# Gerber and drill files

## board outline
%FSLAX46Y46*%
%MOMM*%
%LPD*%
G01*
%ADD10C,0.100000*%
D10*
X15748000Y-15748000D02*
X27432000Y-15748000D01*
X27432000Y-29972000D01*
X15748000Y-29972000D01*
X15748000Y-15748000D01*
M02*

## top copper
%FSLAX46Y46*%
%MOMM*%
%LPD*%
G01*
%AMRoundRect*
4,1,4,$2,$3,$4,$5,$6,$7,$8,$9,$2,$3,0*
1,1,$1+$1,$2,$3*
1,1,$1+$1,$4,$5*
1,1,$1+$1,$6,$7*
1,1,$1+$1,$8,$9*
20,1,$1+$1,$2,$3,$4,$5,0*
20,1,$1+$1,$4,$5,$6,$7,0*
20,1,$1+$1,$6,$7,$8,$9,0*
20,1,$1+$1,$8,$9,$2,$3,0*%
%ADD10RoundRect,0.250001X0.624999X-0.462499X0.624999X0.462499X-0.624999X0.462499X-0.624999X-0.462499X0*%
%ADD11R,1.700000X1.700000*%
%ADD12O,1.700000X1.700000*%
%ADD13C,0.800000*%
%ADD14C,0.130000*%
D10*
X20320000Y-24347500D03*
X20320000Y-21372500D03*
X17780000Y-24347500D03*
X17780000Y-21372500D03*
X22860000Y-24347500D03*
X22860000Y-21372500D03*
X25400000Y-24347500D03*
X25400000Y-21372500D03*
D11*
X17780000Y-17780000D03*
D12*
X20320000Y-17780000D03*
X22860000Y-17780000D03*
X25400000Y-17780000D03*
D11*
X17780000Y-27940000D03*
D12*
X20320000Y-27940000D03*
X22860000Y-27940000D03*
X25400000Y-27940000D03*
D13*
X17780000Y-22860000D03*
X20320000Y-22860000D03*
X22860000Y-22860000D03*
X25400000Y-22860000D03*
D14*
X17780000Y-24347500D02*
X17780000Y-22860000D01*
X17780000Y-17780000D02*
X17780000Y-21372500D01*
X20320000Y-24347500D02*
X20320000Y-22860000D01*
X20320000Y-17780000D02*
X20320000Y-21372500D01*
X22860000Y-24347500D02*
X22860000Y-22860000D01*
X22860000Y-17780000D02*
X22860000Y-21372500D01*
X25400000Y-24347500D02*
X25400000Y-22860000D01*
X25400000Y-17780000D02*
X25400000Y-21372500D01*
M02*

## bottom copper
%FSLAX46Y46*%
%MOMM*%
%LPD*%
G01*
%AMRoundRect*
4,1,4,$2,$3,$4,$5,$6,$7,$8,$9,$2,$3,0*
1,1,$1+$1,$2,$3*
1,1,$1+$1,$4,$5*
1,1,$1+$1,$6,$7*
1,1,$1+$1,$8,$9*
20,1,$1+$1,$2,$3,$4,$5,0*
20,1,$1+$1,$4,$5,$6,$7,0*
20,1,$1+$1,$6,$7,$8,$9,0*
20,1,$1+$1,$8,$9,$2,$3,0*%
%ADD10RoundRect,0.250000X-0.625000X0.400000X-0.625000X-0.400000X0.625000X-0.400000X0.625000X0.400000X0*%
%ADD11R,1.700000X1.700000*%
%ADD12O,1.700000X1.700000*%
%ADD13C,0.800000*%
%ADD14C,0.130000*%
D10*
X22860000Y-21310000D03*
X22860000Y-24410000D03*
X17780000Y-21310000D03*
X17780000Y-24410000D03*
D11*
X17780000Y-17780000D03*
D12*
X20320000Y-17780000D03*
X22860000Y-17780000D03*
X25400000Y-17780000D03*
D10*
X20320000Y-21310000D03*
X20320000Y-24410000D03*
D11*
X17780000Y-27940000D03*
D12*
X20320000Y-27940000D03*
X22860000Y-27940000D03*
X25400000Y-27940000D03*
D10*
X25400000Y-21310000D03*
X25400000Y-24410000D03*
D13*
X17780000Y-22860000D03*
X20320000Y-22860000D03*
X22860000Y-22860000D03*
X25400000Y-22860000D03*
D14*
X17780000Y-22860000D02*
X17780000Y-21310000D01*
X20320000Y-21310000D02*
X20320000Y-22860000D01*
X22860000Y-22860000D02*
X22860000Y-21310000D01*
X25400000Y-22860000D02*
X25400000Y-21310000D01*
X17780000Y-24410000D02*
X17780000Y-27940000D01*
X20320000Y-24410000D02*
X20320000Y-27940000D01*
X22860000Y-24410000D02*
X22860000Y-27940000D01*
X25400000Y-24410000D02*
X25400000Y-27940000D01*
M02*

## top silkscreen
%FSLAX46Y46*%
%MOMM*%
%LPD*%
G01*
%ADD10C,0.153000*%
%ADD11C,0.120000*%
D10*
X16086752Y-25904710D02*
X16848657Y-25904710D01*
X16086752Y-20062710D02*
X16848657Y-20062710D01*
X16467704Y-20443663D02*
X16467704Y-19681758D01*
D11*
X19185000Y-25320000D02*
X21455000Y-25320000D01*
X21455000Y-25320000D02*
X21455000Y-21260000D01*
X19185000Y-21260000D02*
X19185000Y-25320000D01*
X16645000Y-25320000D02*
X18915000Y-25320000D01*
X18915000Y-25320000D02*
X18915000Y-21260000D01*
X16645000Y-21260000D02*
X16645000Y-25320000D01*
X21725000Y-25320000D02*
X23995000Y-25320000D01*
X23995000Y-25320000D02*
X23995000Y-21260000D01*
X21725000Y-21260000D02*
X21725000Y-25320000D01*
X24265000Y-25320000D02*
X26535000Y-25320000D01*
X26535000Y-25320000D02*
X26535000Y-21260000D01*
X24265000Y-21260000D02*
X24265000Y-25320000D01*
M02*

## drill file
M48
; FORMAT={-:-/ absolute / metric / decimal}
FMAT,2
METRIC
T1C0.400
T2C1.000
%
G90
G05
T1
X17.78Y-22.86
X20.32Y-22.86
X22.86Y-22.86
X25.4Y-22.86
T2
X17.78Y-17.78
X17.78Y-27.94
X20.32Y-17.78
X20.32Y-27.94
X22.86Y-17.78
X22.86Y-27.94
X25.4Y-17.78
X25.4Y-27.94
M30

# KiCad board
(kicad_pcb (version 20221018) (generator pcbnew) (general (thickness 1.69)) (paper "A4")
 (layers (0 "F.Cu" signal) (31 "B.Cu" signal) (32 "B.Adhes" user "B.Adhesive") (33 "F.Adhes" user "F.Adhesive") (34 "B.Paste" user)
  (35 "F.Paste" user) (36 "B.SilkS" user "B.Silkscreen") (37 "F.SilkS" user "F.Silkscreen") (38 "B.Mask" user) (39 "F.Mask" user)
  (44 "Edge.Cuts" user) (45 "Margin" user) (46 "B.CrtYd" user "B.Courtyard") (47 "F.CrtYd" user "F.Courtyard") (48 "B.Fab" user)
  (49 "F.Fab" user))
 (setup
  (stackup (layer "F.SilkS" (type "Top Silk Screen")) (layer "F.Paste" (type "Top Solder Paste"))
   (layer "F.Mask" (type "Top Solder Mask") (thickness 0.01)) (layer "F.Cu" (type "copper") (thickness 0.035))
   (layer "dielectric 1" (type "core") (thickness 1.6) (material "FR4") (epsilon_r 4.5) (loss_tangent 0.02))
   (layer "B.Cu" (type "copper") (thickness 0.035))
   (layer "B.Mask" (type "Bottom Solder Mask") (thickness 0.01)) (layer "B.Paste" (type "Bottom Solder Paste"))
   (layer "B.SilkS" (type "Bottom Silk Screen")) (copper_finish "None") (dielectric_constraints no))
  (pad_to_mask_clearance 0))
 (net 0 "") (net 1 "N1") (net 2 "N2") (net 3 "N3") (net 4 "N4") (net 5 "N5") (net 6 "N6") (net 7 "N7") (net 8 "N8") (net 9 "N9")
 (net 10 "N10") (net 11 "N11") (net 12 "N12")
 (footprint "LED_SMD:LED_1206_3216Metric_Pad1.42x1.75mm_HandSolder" (layer "F.Cu") (at 20.32 22.86 90)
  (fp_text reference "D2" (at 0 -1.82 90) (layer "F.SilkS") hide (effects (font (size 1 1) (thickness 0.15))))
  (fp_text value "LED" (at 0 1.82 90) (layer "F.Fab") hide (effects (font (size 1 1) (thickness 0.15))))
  (fp_line (start -2.46 -1.135) (end -2.46 1.135) (stroke (width 0.12) (type solid)) (layer "F.SilkS"))
  (fp_line (start -2.46 1.135) (end 1.6 1.135) (stroke (width 0.12) (type solid)) (layer "F.SilkS"))
  (fp_line (start 1.6 -1.135) (end -2.46 -1.135) (stroke (width 0.12) (type solid)) (layer "F.SilkS"))
  (pad "1" smd roundrect (at -1.4875 0 90) (size 1.425 1.75) (layers "F.Cu" "F.Paste" "F.Mask") (roundrect_rratio 0.1754392982) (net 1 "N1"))
  (pad "2" smd roundrect (at 1.4875 0 90) (size 1.425 1.75) (layers "F.Cu" "F.Paste" "F.Mask") (roundrect_rratio 0.1754392982) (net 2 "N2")))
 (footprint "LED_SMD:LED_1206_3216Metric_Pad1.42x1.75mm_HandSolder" (layer "F.Cu") (at 17.78 22.86 90)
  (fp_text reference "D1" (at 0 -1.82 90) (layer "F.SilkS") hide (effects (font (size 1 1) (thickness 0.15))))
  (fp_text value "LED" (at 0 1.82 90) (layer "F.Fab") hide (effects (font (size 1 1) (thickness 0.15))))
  (fp_line (start -2.46 -1.135) (end -2.46 1.135) (stroke (width 0.12) (type solid)) (layer "F.SilkS"))
  (fp_line (start -2.46 1.135) (end 1.6 1.135) (stroke (width 0.12) (type solid)) (layer "F.SilkS"))
  (fp_line (start 1.6 -1.135) (end -2.46 -1.135) (stroke (width 0.12) (type solid)) (layer "F.SilkS"))
  (pad "1" smd roundrect (at -1.4875 0 90) (size 1.425 1.75) (layers "F.Cu" "F.Paste" "F.Mask") (roundrect_rratio 0.1754392982) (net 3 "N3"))
  (pad "2" smd roundrect (at 1.4875 0 90) (size 1.425 1.75) (layers "F.Cu" "F.Paste" "F.Mask") (roundrect_rratio 0.1754392982) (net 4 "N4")))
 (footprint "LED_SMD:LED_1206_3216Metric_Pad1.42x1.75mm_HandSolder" (layer "F.Cu") (at 22.86 22.86 90)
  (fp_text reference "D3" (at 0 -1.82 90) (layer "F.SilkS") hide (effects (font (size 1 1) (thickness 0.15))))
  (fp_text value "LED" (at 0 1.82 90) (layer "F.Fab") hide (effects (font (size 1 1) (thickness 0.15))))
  (fp_line (start -2.46 -1.135) (end -2.46 1.135) (stroke (width 0.12) (type solid)) (layer "F.SilkS"))
  (fp_line (start -2.46 1.135) (end 1.6 1.135) (stroke (width 0.12) (type solid)) (layer "F.SilkS"))
  (fp_line (start 1.6 -1.135) (end -2.46 -1.135) (stroke (width 0.12) (type solid)) (layer "F.SilkS"))
  (pad "1" smd roundrect (at -1.4875 0 90) (size 1.425 1.75) (layers "F.Cu" "F.Paste" "F.Mask") (roundrect_rratio 0.1754392982) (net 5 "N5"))
  (pad "2" smd roundrect (at 1.4875 0 90) (size 1.425 1.75) (layers "F.Cu" "F.Paste" "F.Mask") (roundrect_rratio 0.1754392982) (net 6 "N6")))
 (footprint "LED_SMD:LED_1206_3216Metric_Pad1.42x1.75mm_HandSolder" (layer "F.Cu") (at 25.4 22.86 90)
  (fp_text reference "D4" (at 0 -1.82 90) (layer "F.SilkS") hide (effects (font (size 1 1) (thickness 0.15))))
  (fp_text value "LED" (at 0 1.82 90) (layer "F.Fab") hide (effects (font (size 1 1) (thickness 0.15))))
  (fp_line (start -2.46 -1.135) (end -2.46 1.135) (stroke (width 0.12) (type solid)) (layer "F.SilkS"))
  (fp_line (start -2.46 1.135) (end 1.6 1.135) (stroke (width 0.12) (type solid)) (layer "F.SilkS"))
  (fp_line (start 1.6 -1.135) (end -2.46 -1.135) (stroke (width 0.12) (type solid)) (layer "F.SilkS"))
  (pad "1" smd roundrect (at -1.4875 0 90) (size 1.425 1.75) (layers "F.Cu" "F.Paste" "F.Mask") (roundrect_rratio 0.1754392982) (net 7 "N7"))
  (pad "2" smd roundrect (at 1.4875 0 90) (size 1.425 1.75) (layers "F.Cu" "F.Paste" "F.Mask") (roundrect_rratio 0.1754392982) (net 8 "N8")))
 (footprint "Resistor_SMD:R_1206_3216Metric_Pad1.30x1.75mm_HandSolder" (layer "B.Cu") (at 22.86 22.86 -90)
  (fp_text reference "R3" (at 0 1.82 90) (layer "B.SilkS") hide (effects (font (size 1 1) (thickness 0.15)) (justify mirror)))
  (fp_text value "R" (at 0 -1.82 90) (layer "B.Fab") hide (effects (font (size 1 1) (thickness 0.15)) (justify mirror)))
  (pad "1" smd roundrect (at -1.55 0 270) (size 1.3 1.75) (layers "B.Cu" "B.Paste" "B.Mask") (roundrect_rratio 0.1923076923) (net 5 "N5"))
  (pad "2" smd roundrect (at 1.55 0 270) (size 1.3 1.75) (layers "B.Cu" "B.Paste" "B.Mask") (roundrect_rratio 0.1923076923) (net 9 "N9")))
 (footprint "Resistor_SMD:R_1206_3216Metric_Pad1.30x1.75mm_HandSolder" (layer "B.Cu") (at 17.78 22.86 -90)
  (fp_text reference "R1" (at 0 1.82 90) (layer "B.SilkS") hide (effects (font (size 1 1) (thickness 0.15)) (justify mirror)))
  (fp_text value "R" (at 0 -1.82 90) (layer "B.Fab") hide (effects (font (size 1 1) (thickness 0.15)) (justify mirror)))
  (pad "1" smd roundrect (at -1.55 0 270) (size 1.3 1.75) (layers "B.Cu" "B.Paste" "B.Mask") (roundrect_rratio 0.1923076923) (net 3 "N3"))
  (pad "2" smd roundrect (at 1.55 0 270) (size 1.3 1.75) (layers "B.Cu" "B.Paste" "B.Mask") (roundrect_rratio 0.1923076923) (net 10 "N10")))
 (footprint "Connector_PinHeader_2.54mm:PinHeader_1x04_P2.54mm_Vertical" (layer "B.Cu") (at 17.78 17.78 -90)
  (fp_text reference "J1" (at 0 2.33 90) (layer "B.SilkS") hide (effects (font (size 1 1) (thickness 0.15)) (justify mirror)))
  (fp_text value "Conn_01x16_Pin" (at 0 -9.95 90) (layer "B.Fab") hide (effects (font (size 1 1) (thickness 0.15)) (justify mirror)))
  (pad "1" thru_hole rect (at 0 0 270) (size 1.7 1.7) (drill 1) (layers "*.Cu" "*.Mask") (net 4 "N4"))
  (pad "2" thru_hole oval (at 0 -2.54 270) (size 1.7 1.7) (drill 1) (layers "*.Cu" "*.Mask") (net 2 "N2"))
  (pad "3" thru_hole oval (at 0 -5.08 270) (size 1.7 1.7) (drill 1) (layers "*.Cu" "*.Mask") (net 6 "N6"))
  (pad "4" thru_hole oval (at 0 -7.62 270) (size 1.7 1.7) (drill 1) (layers "*.Cu" "*.Mask") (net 8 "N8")))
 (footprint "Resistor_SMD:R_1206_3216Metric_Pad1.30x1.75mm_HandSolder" (layer "B.Cu") (at 20.32 22.86 -90)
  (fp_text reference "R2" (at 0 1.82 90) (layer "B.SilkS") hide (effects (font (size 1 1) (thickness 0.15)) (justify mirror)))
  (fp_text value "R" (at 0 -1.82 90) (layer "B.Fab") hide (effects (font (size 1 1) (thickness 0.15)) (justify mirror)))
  (pad "1" smd roundrect (at -1.55 0 270) (size 1.3 1.75) (layers "B.Cu" "B.Paste" "B.Mask") (roundrect_rratio 0.1923076923) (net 1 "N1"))
  (pad "2" smd roundrect (at 1.55 0 270) (size 1.3 1.75) (layers "B.Cu" "B.Paste" "B.Mask") (roundrect_rratio 0.1923076923) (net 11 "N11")))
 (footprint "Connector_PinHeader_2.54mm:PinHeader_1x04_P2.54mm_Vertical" (layer "B.Cu") (at 17.78 27.94 -90)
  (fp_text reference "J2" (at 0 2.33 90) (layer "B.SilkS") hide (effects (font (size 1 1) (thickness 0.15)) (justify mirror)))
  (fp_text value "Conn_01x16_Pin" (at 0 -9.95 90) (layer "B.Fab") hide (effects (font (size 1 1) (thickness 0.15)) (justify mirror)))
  (pad "1" thru_hole rect (at 0 0 270) (size 1.7 1.7) (drill 1) (layers "*.Cu" "*.Mask") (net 10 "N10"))
  (pad "2" thru_hole oval (at 0 -2.54 270) (size 1.7 1.7) (drill 1) (layers "*.Cu" "*.Mask") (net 11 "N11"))
  (pad "3" thru_hole oval (at 0 -5.08 270) (size 1.7 1.7) (drill 1) (layers "*.Cu" "*.Mask") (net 9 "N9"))
  (pad "4" thru_hole oval (at 0 -7.62 270) (size 1.7 1.7) (drill 1) (layers "*.Cu" "*.Mask") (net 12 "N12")))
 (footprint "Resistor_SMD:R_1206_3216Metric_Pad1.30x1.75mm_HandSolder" (layer "B.Cu") (at 25.4 22.86 -90)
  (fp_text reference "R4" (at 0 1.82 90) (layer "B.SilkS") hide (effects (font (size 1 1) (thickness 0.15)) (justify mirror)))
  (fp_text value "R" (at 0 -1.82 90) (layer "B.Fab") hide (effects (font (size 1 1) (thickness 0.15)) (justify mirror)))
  (pad "1" smd roundrect (at -1.55 0 270) (size 1.3 1.75) (layers "B.Cu" "B.Paste" "B.Mask") (roundrect_rratio 0.1923076923) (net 7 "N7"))
  (pad "2" smd roundrect (at 1.55 0 270) (size 1.3 1.75) (layers "B.Cu" "B.Paste" "B.Mask") (roundrect_rratio 0.1923076923) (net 12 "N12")))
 (gr_rect (start 15.748 15.748) (end 27.432 29.972) (stroke (width 0.1) (type default)) (fill none) (layer "Edge.Cuts"))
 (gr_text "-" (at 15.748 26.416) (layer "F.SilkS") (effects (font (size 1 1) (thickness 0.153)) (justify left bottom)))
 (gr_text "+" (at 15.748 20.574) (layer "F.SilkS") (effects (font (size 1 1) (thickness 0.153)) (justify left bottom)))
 (segment (start 17.78 24.3475) (end 17.78 22.86) (width 0.13) (layer "F.Cu") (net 3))
 (via (at 17.78 22.86) (size 0.8) (drill 0.4) (layers "F.Cu" "B.Cu") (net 3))
 (segment (start 17.78 22.86) (end 17.78 21.31) (width 0.13) (layer "B.Cu") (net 3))
 (segment (start 17.78 17.78) (end 17.78 21.3725) (width 0.13) (layer "F.Cu") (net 4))
 (segment (start 20.32 24.3475) (end 20.32 22.86) (width 0.13) (layer "F.Cu") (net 1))
 (via (at 20.32 22.86) (size 0.8) (drill 0.4) (layers "F.Cu" "B.Cu") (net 1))
 (segment (start 20.32 21.31) (end 20.32 22.86) (width 0.13) (layer "B.Cu") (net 1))
 (segment (start 20.32 17.78) (end 20.32 21.3725) (width 0.13) (layer "F.Cu") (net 2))
 (segment (start 22.86 24.3475) (end 22.86 22.86) (width 0.13) (layer "F.Cu") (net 5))
 (via (at 22.86 22.86) (size 0.8) (drill 0.4) (layers "F.Cu" "B.Cu") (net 5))
 (segment (start 22.86 22.86) (end 22.86 21.31) (width 0.13) (layer "B.Cu") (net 5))
 (segment (start 22.86 17.78) (end 22.86 21.3725) (width 0.13) (layer "F.Cu") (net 6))
 (segment (start 25.4 24.3475) (end 25.4 22.86) (width 0.13) (layer "F.Cu") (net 7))
 (via (at 25.4 22.86) (size 0.8) (drill 0.4) (layers "F.Cu" "B.Cu") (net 7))
 (segment (start 25.4 22.86) (end 25.4 21.31) (width 0.13) (layer "B.Cu") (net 7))
 (segment (start 25.4 17.78) (end 25.4 21.3725) (width 0.13) (layer "F.Cu") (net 8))
 (segment (start 17.78 24.41) (end 17.78 27.94) (width 0.13) (layer "B.Cu") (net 10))
 (segment (start 20.32 24.41) (end 20.32 27.94) (width 0.13) (layer "B.Cu") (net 11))
 (segment (start 22.86 24.41) (end 22.86 27.94) (width 0.13) (layer "B.Cu") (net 9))
 (segment (start 25.4 24.41) (end 25.4 27.94) (width 0.13) (layer "B.Cu") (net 12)))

